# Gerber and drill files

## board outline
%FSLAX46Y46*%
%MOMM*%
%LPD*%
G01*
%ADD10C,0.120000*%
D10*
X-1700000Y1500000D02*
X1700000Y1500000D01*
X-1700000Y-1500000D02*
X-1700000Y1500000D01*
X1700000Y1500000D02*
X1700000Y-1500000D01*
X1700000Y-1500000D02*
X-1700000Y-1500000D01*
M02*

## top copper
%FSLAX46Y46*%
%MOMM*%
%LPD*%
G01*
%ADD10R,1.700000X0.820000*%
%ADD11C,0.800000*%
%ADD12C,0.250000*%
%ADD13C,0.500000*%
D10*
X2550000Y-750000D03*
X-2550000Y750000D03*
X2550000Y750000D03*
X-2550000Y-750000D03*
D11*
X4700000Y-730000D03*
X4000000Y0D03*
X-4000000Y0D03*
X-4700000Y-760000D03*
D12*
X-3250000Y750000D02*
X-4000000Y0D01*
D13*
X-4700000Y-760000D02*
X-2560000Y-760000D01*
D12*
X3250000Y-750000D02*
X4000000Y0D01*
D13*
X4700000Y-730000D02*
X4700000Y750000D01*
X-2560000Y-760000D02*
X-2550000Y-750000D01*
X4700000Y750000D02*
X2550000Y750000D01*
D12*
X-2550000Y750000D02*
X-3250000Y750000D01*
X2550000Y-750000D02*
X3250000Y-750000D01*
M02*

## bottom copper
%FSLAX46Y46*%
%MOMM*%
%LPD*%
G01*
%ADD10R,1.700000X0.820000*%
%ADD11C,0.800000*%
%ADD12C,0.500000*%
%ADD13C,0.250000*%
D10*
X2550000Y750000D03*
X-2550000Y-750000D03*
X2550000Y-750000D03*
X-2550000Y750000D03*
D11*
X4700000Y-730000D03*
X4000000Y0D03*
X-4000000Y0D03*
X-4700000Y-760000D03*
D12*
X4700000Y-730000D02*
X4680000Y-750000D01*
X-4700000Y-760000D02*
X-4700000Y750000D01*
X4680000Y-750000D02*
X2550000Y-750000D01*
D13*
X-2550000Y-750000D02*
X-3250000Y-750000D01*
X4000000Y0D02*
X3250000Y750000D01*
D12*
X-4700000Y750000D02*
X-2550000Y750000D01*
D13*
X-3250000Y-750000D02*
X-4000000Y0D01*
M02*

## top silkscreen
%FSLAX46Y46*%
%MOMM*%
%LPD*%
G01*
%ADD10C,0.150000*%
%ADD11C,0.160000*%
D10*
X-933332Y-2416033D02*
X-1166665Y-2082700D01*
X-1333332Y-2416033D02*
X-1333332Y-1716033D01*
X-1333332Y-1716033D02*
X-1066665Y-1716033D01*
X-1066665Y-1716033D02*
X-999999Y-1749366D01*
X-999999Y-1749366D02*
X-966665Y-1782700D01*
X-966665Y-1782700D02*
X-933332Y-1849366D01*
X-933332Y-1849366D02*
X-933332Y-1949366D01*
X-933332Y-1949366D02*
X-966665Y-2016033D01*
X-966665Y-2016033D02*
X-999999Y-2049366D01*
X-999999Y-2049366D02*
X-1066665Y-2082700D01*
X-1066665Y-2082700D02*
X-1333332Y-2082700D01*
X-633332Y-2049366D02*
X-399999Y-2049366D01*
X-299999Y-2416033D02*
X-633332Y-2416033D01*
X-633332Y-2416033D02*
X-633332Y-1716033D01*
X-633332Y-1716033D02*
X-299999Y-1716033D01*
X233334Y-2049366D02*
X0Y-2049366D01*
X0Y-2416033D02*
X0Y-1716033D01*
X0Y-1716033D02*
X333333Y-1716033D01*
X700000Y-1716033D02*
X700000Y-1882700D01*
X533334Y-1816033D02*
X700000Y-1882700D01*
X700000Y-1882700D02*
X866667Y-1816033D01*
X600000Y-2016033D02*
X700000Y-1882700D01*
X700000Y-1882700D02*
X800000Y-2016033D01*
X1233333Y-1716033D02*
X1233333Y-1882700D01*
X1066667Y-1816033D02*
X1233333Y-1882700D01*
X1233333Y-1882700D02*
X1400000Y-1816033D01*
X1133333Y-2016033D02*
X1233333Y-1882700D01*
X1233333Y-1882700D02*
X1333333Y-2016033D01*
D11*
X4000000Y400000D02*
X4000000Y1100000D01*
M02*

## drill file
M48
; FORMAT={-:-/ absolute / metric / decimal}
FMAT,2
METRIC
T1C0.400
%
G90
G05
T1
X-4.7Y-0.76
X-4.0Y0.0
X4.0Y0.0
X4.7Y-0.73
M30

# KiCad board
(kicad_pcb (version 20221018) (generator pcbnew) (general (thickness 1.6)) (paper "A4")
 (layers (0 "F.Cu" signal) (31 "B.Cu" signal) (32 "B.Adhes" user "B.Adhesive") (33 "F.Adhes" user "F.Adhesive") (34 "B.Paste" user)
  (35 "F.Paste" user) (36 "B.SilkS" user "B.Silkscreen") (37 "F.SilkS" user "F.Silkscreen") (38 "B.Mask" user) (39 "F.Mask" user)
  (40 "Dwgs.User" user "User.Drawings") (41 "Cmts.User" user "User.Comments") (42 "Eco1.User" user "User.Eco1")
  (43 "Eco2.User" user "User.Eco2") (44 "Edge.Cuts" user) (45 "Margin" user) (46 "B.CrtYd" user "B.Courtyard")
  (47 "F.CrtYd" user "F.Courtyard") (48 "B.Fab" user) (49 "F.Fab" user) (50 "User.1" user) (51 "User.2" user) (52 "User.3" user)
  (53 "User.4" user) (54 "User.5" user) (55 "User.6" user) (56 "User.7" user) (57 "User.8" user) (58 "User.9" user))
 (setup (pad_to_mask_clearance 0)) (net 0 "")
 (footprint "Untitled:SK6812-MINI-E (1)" (layer "F.Cu") (at 0 0)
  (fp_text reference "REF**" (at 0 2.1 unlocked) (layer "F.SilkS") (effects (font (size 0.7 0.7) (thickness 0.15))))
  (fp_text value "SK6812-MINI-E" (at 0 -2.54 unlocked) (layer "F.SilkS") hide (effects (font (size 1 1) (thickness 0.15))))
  (fp_line (start 4 -0.4) (end 4 -1.1) (stroke (width 0.16) (type solid)) (layer "F.SilkS"))
  (fp_line (start -1.7 -1.5) (end 1.7 -1.5) (stroke (width 0.12) (type solid)) (layer "Edge.Cuts"))
  (fp_line (start -1.7 1.5) (end -1.7 -1.5) (stroke (width 0.12) (type solid)) (layer "Edge.Cuts"))
  (fp_line (start 1.7 -1.5) (end 1.7 1.5) (stroke (width 0.12) (type solid)) (layer "Edge.Cuts"))
  (fp_line (start 1.7 1.5) (end -1.7 1.5) (stroke (width 0.12) (type solid)) (layer "Edge.Cuts"))
  (pad "DIN" smd rect (at 2.55 -0.75) (size 1.7 0.82) (layers "B.Cu" "B.Paste" "B.Mask"))
  (pad "DIN" smd rect (at 2.55 0.75) (size 1.7 0.82) (layers "F.Cu" "F.Paste" "F.Mask"))
  (pad "DOUT" smd rect (at -2.55 -0.75) (size 1.7 0.82) (layers "F.Cu" "F.Paste" "F.Mask"))
  (pad "DOUT" smd rect (at -2.55 0.75) (size 1.7 0.82) (layers "B.Cu" "B.Paste" "B.Mask"))
  (pad "GND" smd rect (at 2.55 -0.75) (size 1.7 0.82) (layers "F.Cu" "F.Paste" "F.Mask"))
  (pad "GND" smd rect (at 2.55 0.75) (size 1.7 0.82) (layers "B.Cu" "B.Paste" "B.Mask"))
  (pad "VDD" smd rect (at -2.55 -0.75) (size 1.7 0.82) (layers "B.Cu" "B.Paste" "B.Mask"))
  (pad "VDD" smd rect (at -2.55 0.75) (size 1.7 0.82) (layers "F.Cu" "F.Paste" "F.Mask")))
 (segment (start -3.25 -0.75) (end -4 0) (width 0.25) (layer "F.Cu") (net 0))
 (segment (start -4.7 0.76) (end -2.56 0.76) (width 0.5) (layer "F.Cu") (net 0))
 (segment (start 3.25 0.75) (end 4 0) (width 0.25) (layer "F.Cu") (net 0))
 (segment (start 4.7 0.73) (end 4.7 -0.75) (width 0.5) (layer "F.Cu") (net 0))
 (segment (start -2.56 0.76) (end -2.55 0.75) (width 0.5) (layer "F.Cu") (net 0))
 (segment (start 4.7 -0.75) (end 2.55 -0.75) (width 0.5) (layer "F.Cu") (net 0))
 (segment (start -2.55 -0.75) (end -3.25 -0.75) (width 0.25) (layer "F.Cu") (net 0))
 (segment (start 2.55 0.75) (end 3.25 0.75) (width 0.25) (layer "F.Cu") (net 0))
 (via (at 4.7 0.73) (size 0.8) (drill 0.4) (layers "F.Cu" "B.Cu") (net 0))
 (via (at 4 0) (size 0.8) (drill 0.4) (layers "F.Cu" "B.Cu") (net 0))
 (via (at -4 0) (size 0.8) (drill 0.4) (layers "F.Cu" "B.Cu") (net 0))
 (via (at -4.7 0.76) (size 0.8) (drill 0.4) (layers "F.Cu" "B.Cu") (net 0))
 (segment (start 4.7 0.73) (end 4.68 0.75) (width 0.5) (layer "B.Cu") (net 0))
 (segment (start -4.7 0.76) (end -4.7 -0.75) (width 0.5) (layer "B.Cu") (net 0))
 (segment (start 4.68 0.75) (end 2.55 0.75) (width 0.5) (layer "B.Cu") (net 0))
 (segment (start -2.55 0.75) (end -3.25 0.75) (width 0.25) (layer "B.Cu") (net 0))
 (segment (start 4 0) (end 3.25 -0.75) (width 0.25) (layer "B.Cu") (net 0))
 (segment (start -4.7 -0.75) (end -2.55 -0.75) (width 0.5) (layer "B.Cu") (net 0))
 (segment (start -3.25 0.75) (end -4 0) (width 0.25) (layer "B.Cu") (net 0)))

